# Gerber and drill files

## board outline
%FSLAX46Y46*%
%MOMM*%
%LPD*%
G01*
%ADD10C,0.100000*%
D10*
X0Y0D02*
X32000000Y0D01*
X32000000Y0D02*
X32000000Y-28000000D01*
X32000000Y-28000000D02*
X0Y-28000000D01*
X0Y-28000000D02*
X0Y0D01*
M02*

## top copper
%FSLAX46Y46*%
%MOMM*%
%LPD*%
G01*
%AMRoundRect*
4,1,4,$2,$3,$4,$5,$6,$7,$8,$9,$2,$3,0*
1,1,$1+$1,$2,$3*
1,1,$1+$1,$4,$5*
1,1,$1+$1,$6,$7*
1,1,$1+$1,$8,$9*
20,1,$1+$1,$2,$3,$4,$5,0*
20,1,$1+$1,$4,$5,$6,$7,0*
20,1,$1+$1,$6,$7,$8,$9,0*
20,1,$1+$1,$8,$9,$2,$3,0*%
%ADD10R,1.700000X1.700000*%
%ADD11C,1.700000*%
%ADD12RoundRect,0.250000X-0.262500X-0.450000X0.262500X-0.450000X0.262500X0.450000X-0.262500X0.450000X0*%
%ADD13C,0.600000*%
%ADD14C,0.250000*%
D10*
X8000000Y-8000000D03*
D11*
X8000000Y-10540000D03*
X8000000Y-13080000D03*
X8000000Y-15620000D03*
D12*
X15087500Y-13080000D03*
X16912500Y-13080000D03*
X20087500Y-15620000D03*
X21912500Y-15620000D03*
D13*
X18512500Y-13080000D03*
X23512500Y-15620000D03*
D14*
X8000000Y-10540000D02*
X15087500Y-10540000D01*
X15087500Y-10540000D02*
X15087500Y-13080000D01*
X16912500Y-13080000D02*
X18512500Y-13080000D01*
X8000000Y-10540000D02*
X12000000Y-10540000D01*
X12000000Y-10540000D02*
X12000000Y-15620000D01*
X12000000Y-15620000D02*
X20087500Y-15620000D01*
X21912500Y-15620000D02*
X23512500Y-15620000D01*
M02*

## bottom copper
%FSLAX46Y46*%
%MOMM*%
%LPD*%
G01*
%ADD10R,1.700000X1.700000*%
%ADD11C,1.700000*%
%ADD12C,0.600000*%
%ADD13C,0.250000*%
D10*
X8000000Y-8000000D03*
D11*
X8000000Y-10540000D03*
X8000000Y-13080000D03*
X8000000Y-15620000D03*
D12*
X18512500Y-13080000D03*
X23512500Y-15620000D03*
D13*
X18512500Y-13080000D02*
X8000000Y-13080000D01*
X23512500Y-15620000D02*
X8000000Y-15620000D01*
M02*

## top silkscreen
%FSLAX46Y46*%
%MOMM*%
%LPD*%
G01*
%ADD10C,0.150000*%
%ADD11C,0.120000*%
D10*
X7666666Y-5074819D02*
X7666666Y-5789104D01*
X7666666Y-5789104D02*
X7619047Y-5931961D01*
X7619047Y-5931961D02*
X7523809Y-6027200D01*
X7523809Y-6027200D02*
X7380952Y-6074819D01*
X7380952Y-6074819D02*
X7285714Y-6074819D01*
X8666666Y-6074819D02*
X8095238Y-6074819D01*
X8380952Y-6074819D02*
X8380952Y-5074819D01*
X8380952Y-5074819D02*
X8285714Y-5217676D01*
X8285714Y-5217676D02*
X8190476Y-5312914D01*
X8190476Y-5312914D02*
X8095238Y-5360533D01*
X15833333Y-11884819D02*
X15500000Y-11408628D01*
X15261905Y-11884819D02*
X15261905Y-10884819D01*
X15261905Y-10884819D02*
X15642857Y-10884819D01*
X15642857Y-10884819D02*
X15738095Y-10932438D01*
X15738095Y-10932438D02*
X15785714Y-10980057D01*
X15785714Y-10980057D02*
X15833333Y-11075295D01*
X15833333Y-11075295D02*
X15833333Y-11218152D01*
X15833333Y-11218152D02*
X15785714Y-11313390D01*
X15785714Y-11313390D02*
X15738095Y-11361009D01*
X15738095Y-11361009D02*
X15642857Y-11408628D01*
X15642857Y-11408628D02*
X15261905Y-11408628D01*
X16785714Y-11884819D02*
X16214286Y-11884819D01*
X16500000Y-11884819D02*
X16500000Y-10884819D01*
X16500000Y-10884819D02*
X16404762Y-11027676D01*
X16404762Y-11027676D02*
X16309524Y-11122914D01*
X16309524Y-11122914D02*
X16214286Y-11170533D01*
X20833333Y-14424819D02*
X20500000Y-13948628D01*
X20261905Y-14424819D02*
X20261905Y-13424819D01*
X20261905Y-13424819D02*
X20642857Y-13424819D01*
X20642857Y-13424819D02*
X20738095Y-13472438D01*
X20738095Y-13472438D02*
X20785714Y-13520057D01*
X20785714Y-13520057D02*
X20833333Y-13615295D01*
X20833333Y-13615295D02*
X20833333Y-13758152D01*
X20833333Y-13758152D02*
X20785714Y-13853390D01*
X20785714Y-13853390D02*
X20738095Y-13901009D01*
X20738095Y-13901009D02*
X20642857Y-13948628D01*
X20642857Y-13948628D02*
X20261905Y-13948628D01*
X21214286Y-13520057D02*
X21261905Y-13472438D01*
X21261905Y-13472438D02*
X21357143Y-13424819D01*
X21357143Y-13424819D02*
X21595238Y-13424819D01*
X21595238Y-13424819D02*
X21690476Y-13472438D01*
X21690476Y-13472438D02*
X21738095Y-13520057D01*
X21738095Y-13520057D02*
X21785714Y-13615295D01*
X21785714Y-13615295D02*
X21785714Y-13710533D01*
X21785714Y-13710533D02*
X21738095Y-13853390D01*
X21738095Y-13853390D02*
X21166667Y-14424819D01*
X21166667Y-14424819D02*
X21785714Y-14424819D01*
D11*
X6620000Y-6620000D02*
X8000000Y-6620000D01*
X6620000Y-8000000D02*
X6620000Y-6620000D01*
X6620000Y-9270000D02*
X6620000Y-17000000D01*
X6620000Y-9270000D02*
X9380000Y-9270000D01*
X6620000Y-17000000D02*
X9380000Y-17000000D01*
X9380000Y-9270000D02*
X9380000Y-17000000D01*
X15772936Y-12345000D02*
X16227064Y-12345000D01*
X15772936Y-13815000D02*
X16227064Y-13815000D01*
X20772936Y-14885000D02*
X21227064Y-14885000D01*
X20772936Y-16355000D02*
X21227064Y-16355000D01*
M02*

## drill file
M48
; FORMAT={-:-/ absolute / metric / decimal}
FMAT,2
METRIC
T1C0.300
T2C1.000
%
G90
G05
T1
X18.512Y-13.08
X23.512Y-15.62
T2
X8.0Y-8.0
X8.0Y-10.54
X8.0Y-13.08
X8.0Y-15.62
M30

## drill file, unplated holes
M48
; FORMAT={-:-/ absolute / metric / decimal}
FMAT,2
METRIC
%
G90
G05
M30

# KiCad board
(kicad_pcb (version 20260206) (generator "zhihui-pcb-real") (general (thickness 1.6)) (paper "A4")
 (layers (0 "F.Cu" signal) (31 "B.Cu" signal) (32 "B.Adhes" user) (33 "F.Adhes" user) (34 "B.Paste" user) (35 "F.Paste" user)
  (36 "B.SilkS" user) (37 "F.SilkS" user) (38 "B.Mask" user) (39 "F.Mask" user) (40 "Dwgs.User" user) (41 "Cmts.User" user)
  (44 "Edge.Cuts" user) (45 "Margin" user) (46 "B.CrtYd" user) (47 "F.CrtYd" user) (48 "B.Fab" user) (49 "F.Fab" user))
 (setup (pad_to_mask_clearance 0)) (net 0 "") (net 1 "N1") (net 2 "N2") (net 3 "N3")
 (gr_line (start 0 0) (end 32 0) (stroke (width 0.1) (type default)) (layer "Edge.Cuts"))
 (gr_line (start 32 0) (end 32 28) (stroke (width 0.1) (type default)) (layer "Edge.Cuts"))
 (gr_line (start 32 28) (end 0 28) (stroke (width 0.1) (type default)) (layer "Edge.Cuts"))
 (gr_line (start 0 28) (end 0 0) (stroke (width 0.1) (type default)) (layer "Edge.Cuts"))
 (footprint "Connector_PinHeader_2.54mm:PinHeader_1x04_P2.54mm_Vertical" (layer "F.Cu")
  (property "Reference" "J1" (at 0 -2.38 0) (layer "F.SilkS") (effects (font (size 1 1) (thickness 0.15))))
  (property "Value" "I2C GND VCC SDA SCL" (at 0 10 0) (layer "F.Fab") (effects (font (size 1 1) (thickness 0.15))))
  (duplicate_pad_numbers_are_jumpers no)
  (fp_line (start -1.38 -1.38) (end 0 -1.38) (stroke (width 0.12) (type solid)) (layer "F.SilkS"))
  (fp_line (start -1.38 0) (end -1.38 -1.38) (stroke (width 0.12) (type solid)) (layer "F.SilkS"))
  (fp_line (start -1.38 1.27) (end -1.38 9) (stroke (width 0.12) (type solid)) (layer "F.SilkS"))
  (fp_line (start -1.38 1.27) (end 1.38 1.27) (stroke (width 0.12) (type solid)) (layer "F.SilkS"))
  (fp_line (start -1.38 9) (end 1.38 9) (stroke (width 0.12) (type solid)) (layer "F.SilkS"))
  (fp_line (start 1.38 1.27) (end 1.38 9) (stroke (width 0.12) (type solid)) (layer "F.SilkS"))
  (pad "1" thru_hole rect (at 0 0) (size 1.7 1.7) (drill 1) (layers "*.Cu" "*.Mask") (remove_unused_layers no))
  (pad "2" thru_hole circle (at 0 2.54) (size 1.7 1.7) (drill 1) (layers "*.Cu" "*.Mask") (remove_unused_layers no) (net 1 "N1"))
  (pad "3" thru_hole circle (at 0 5.08) (size 1.7 1.7) (drill 1) (layers "*.Cu" "*.Mask") (remove_unused_layers no) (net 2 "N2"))
  (pad "4" thru_hole circle (at 0 7.62) (size 1.7 1.7) (drill 1) (layers "*.Cu" "*.Mask") (remove_unused_layers no) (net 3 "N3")) (at 8 8 0))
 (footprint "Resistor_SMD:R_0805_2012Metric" (layer "F.Cu")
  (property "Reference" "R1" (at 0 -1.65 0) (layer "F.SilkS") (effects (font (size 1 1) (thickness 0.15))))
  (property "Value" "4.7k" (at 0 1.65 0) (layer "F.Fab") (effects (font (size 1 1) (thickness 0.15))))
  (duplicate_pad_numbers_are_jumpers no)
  (fp_line (start -0.227064 -0.735) (end 0.227064 -0.735) (stroke (width 0.12) (type solid)) (layer "F.SilkS"))
  (fp_line (start -0.227064 0.735) (end 0.227064 0.735) (stroke (width 0.12) (type solid)) (layer "F.SilkS"))
  (pad "1" smd roundrect (at -0.9125 0) (size 1.025 1.4) (layers "F.Cu" "F.Mask" "F.Paste") (roundrect_rratio 0.243902) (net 1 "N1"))
  (pad "2" smd roundrect (at 0.9125 0) (size 1.025 1.4) (layers "F.Cu" "F.Mask" "F.Paste") (roundrect_rratio 0.243902) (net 2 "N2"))
  (at 16 13.08 0))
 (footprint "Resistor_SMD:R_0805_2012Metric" (layer "F.Cu")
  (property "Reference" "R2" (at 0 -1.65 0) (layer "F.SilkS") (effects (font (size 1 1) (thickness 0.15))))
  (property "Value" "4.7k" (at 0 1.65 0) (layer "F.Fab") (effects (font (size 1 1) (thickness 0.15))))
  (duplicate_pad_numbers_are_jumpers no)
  (fp_line (start -0.227064 -0.735) (end 0.227064 -0.735) (stroke (width 0.12) (type solid)) (layer "F.SilkS"))
  (fp_line (start -0.227064 0.735) (end 0.227064 0.735) (stroke (width 0.12) (type solid)) (layer "F.SilkS"))
  (pad "1" smd roundrect (at -0.9125 0) (size 1.025 1.4) (layers "F.Cu" "F.Mask" "F.Paste") (roundrect_rratio 0.243902) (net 1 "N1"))
  (pad "2" smd roundrect (at 0.9125 0) (size 1.025 1.4) (layers "F.Cu" "F.Mask" "F.Paste") (roundrect_rratio 0.243902) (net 3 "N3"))
  (at 21 15.62 0))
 (segment (start 8 10.54) (end 15.0875 10.54) (width 0.25) (layer "F.Cu") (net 1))
 (segment (start 15.0875 10.54) (end 15.0875 13.08) (width 0.25) (layer "F.Cu") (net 1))
 (segment (start 16.9125 13.08) (end 18.5125 13.08) (width 0.25) (layer "F.Cu") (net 2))
 (segment (start 18.5125 13.08) (end 8 13.08) (width 0.25) (layer "B.Cu") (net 2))
 (segment (start 8 10.54) (end 12 10.54) (width 0.25) (layer "F.Cu") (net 1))
 (segment (start 12 10.54) (end 12 15.62) (width 0.25) (layer "F.Cu") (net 1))
 (segment (start 12 15.62) (end 20.0875 15.62) (width 0.25) (layer "F.Cu") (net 1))
 (segment (start 21.9125 15.62) (end 23.5125 15.62) (width 0.25) (layer "F.Cu") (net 3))
 (segment (start 23.5125 15.62) (end 8 15.62) (width 0.25) (layer "B.Cu") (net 3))
 (via (at 18.5125 13.08) (size 0.6) (drill 0.3) (layers "F.Cu" "B.Cu") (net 2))
 (via (at 23.5125 15.62) (size 0.6) (drill 0.3) (layers "F.Cu" "B.Cu") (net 3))
 (segment (start 8 8) (end 8 10.54) (width 0.25) (layer "F.Cu") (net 1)))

